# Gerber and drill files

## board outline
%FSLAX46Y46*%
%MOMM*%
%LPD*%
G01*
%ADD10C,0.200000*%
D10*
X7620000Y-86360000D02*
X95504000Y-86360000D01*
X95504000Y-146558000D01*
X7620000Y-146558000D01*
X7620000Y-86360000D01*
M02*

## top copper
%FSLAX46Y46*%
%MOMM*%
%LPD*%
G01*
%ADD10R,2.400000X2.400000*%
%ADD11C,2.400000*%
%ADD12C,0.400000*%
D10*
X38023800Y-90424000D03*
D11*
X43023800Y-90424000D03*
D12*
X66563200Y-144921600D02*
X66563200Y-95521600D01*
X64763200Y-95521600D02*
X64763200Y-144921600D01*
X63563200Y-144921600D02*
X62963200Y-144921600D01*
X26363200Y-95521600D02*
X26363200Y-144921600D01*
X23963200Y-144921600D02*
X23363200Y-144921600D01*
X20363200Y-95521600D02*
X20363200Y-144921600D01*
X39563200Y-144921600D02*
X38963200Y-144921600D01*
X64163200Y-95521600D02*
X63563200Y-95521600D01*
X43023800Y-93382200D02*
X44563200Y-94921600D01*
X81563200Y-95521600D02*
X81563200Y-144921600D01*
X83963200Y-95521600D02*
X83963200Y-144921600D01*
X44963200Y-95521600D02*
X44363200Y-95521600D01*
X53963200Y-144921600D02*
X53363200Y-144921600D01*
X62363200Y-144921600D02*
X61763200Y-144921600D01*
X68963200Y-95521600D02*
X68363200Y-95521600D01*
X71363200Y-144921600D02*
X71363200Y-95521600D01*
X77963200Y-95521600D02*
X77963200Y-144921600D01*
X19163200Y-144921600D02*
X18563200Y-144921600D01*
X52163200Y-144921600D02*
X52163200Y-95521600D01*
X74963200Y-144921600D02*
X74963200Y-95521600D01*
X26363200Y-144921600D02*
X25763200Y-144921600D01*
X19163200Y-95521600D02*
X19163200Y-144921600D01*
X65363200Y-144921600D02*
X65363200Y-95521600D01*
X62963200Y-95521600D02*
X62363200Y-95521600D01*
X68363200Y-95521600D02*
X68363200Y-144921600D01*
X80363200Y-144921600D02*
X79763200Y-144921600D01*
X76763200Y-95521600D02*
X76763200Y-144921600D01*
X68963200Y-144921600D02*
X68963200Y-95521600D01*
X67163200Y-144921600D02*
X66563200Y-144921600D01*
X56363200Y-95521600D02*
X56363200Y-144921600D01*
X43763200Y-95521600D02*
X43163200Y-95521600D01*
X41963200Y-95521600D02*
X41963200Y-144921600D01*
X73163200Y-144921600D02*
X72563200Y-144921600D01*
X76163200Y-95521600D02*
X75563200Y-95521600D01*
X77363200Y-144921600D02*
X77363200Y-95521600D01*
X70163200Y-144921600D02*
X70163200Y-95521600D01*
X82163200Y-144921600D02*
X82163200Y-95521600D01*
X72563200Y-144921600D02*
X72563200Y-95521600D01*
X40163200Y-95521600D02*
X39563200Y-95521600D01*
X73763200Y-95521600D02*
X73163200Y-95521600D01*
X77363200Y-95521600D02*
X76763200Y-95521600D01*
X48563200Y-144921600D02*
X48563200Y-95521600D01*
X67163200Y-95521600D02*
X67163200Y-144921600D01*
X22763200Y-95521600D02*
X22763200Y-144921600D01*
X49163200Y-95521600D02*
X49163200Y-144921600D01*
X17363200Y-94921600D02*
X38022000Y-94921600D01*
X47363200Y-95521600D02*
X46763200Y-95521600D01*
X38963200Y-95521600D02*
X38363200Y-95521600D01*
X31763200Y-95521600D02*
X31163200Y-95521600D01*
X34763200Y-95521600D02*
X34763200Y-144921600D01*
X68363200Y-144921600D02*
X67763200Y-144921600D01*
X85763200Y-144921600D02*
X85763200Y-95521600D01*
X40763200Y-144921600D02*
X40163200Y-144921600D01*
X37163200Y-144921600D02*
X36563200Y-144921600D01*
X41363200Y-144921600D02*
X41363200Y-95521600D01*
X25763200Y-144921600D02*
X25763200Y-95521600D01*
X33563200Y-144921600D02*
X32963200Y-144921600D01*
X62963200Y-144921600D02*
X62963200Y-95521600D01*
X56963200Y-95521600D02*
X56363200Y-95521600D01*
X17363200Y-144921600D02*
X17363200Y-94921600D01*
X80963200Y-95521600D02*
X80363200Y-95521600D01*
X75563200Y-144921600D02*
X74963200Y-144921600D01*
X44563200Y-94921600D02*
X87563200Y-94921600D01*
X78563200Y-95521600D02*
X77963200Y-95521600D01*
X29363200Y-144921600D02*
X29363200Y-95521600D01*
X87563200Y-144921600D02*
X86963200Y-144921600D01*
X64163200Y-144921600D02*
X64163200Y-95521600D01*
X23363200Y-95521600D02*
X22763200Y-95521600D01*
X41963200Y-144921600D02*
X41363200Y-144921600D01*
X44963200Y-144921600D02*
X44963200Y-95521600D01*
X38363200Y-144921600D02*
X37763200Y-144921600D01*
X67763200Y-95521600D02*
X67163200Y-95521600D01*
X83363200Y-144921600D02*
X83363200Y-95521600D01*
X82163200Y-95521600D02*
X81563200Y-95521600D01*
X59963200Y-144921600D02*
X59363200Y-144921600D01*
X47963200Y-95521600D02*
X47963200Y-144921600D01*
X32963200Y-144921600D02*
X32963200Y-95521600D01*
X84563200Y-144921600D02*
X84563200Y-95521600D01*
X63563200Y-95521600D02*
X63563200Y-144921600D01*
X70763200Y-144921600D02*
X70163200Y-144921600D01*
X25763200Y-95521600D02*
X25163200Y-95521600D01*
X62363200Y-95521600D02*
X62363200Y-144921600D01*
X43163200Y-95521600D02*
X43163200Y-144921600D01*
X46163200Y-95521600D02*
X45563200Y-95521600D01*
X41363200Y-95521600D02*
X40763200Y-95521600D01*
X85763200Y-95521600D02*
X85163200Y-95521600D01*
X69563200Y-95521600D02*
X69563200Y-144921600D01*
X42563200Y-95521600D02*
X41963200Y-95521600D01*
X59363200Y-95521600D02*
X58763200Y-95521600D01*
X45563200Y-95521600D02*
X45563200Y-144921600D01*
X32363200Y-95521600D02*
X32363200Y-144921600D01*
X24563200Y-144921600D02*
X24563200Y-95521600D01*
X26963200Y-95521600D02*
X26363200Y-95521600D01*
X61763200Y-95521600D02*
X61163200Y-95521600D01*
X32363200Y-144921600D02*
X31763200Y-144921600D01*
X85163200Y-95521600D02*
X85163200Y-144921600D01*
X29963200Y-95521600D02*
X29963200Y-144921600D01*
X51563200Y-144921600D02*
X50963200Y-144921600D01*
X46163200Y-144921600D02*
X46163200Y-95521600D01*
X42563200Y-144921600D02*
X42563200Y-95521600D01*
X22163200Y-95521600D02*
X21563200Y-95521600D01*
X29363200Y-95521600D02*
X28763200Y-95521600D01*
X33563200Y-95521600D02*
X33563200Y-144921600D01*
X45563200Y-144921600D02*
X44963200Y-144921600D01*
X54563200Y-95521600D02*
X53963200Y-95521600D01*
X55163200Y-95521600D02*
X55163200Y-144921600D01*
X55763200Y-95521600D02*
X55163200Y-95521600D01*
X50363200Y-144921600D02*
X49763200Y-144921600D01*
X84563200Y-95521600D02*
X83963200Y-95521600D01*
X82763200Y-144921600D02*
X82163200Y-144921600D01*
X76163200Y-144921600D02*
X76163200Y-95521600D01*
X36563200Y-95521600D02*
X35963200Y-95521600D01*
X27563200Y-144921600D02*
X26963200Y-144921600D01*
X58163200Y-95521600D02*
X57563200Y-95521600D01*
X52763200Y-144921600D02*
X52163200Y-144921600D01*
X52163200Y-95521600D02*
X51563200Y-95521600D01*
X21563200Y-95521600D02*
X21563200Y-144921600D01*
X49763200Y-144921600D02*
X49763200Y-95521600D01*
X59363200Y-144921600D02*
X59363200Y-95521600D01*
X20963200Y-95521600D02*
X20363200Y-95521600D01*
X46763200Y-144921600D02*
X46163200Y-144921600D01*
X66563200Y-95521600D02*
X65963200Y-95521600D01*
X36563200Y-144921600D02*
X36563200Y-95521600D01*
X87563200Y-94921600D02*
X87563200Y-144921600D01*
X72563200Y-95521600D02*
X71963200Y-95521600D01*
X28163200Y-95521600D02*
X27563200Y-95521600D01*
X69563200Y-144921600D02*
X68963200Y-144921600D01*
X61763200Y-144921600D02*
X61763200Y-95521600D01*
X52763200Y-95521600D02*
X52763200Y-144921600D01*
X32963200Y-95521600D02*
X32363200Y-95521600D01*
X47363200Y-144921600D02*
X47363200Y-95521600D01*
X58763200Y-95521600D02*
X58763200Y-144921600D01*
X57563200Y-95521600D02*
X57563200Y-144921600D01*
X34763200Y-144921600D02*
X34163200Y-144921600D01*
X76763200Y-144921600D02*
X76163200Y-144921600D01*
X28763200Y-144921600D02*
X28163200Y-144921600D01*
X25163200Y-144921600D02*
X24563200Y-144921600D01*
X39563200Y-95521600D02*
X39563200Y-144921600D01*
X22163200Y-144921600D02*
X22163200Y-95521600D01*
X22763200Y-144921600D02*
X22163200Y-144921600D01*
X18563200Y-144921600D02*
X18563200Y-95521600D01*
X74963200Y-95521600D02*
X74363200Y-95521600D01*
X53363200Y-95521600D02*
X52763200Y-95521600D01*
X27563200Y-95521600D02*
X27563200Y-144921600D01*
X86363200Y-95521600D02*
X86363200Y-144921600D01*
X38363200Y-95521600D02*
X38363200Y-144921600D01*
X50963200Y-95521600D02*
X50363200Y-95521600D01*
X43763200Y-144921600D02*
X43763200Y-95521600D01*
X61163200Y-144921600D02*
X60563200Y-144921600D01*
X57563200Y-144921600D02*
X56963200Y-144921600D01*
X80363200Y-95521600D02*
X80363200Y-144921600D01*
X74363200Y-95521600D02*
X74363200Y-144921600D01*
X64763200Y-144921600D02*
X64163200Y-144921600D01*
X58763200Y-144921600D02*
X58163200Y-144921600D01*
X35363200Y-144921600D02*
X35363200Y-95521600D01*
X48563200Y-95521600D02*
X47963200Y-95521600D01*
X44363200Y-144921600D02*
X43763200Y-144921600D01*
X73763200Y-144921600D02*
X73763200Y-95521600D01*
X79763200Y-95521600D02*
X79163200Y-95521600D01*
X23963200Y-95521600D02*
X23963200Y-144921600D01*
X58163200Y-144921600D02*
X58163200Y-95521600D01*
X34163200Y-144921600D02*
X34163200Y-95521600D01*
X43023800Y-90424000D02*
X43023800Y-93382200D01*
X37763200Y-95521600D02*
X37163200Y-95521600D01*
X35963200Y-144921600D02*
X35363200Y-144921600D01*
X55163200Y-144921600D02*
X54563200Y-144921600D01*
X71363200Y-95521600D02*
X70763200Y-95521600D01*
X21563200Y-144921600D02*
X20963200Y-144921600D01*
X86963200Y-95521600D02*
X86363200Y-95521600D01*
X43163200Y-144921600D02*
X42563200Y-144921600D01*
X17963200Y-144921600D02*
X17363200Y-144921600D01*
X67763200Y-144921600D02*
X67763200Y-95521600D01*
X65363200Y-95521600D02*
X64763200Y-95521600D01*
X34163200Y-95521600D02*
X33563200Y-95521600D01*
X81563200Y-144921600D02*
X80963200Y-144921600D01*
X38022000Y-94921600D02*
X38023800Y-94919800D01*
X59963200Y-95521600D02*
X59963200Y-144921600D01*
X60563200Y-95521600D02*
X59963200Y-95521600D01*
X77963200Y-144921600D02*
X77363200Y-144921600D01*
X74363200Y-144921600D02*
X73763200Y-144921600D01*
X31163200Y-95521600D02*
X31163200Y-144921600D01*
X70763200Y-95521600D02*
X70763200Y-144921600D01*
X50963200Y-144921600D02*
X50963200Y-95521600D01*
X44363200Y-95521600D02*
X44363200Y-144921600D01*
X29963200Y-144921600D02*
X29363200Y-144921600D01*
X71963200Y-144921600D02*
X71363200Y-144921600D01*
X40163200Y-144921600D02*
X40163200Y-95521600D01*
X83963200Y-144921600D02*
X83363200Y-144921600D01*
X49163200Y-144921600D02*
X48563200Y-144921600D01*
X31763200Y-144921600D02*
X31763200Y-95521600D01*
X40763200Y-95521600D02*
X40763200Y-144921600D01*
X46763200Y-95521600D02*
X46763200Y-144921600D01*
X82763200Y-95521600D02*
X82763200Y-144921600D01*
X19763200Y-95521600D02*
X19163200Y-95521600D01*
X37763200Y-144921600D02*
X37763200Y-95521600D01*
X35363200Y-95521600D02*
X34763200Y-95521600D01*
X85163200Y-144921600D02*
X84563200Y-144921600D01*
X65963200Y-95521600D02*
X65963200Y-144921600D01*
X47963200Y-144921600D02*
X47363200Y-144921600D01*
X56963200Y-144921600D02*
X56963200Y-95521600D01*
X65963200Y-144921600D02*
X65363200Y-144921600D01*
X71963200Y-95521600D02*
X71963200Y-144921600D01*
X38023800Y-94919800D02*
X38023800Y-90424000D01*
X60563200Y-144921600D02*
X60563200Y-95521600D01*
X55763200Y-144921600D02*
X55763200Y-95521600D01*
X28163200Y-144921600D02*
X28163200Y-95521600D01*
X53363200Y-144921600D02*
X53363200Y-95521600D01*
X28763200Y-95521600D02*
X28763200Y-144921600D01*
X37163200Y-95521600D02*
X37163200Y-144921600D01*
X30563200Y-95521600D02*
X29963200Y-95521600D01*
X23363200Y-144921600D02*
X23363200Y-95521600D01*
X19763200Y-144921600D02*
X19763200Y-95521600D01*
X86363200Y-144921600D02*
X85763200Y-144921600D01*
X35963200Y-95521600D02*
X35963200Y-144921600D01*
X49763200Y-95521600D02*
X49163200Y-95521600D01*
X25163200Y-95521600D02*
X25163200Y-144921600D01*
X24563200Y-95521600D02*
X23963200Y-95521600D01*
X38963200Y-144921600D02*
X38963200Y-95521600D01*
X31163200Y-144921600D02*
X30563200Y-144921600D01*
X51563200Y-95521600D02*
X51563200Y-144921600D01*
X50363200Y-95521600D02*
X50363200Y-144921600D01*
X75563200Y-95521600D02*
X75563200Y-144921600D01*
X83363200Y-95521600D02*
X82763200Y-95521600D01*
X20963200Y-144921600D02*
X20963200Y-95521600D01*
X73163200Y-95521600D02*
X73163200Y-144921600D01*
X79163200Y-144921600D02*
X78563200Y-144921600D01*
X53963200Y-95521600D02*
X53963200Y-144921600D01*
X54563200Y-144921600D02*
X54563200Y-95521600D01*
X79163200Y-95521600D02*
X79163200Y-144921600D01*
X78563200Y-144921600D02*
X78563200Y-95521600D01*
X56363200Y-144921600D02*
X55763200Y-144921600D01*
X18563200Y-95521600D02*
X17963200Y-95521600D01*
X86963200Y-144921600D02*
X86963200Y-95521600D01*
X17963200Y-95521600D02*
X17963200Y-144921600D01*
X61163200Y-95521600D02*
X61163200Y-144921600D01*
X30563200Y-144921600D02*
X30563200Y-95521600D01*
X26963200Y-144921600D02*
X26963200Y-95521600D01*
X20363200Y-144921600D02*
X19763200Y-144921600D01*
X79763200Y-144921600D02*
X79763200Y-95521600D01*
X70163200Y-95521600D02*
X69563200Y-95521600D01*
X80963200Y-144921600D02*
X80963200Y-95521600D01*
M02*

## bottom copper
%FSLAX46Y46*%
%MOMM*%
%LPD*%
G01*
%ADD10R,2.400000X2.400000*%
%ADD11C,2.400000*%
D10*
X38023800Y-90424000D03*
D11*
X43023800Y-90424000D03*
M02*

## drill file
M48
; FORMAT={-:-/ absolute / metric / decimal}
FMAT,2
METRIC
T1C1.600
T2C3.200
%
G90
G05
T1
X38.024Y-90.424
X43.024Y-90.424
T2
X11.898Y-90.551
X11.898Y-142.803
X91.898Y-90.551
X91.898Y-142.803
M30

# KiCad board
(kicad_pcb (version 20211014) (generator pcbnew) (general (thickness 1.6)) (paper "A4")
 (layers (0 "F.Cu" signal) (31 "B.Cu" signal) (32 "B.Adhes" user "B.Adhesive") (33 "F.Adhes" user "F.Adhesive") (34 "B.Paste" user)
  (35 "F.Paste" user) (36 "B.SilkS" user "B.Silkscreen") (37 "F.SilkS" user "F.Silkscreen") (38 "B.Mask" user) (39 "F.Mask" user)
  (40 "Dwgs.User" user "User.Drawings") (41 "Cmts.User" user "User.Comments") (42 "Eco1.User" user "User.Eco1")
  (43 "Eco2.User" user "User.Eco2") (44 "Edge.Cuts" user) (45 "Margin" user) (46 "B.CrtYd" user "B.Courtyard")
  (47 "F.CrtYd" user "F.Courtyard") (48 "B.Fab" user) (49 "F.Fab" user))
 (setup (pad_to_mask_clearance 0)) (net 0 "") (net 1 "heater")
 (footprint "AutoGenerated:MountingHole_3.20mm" (layer "F.Cu") (at 91.898 142.803)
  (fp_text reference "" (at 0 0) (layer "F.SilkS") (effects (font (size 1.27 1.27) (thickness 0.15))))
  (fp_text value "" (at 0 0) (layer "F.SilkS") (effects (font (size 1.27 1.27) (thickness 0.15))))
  (pad "" np_thru_hole circle locked (at 0 0) (size 3.2 3.2) (drill 3.2) (layers *.Cu *.Mask)))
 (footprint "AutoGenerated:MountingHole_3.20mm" (layer "F.Cu") (at 11.898 90.551)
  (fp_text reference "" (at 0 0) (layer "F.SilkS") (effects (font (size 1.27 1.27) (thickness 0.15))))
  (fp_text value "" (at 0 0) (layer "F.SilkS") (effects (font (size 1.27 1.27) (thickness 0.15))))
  (pad "" np_thru_hole circle locked (at 0 0) (size 3.2 3.2) (drill 3.2) (layers *.Cu *.Mask)))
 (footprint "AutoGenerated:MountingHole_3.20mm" (layer "F.Cu") (at 91.898 90.551)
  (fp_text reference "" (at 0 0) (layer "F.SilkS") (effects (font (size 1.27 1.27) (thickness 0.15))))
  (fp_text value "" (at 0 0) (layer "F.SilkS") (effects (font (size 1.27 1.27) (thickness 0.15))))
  (pad "" np_thru_hole circle locked (at 0 0) (size 3.2 3.2) (drill 3.2) (layers *.Cu *.Mask)))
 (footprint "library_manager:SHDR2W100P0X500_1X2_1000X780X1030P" (layer "F.Cu") (at 38.0238 90.424)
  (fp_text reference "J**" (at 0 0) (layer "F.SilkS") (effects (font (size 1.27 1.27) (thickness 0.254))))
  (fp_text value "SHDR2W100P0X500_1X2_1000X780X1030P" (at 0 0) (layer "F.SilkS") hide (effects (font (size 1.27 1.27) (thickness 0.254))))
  (pad "1" thru_hole rect locked (at 0 0) (size 2.4 2.4) (drill 1.6) (layers *.Cu *.Mask) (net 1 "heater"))
  (pad "2" thru_hole circle locked (at 5 0) (size 2.4 2.4) (drill 1.6) (layers *.Cu *.Mask) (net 1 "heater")))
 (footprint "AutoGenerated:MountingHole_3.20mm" (layer "F.Cu") (at 11.898 142.803)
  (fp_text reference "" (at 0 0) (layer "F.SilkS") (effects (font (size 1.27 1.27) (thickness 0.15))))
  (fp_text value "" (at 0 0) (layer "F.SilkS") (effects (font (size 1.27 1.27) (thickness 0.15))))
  (pad "" np_thru_hole circle locked (at 0 0) (size 3.2 3.2) (drill 3.2) (layers *.Cu *.Mask)))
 (gr_rect (start 7.62 86.36) (end 95.504 146.558) (layer "Edge.Cuts") (width 0.2) (fill none))
 (segment (start 66.5632 144.9216) (end 66.5632 95.5216) (width 0.4) (layer "F.Cu") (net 1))
 (segment (start 64.7632 95.5216) (end 64.7632 144.9216) (width 0.4) (layer "F.Cu") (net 1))
 (segment (start 63.5632 144.9216) (end 62.9632 144.9216) (width 0.4) (layer "F.Cu") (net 1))
 (segment (start 26.3632 95.5216) (end 26.3632 144.9216) (width 0.4) (layer "F.Cu") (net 1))
 (segment (start 23.9632 144.9216) (end 23.3632 144.9216) (width 0.4) (layer "F.Cu") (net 1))
 (segment (start 20.3632 95.5216) (end 20.3632 144.9216) (width 0.4) (layer "F.Cu") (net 1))
 (segment (start 39.5632 144.9216) (end 38.9632 144.9216) (width 0.4) (layer "F.Cu") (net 1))
 (segment (start 64.1632 95.5216) (end 63.5632 95.5216) (width 0.4) (layer "F.Cu") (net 1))
 (segment (start 43.0238 93.3822) (end 44.5632 94.9216) (width 0.4) (layer "F.Cu") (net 1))
 (segment (start 81.5632 95.5216) (end 81.5632 144.9216) (width 0.4) (layer "F.Cu") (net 1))
 (segment (start 83.9632 95.5216) (end 83.9632 144.9216) (width 0.4) (layer "F.Cu") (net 1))
 (segment (start 44.9632 95.5216) (end 44.3632 95.5216) (width 0.4) (layer "F.Cu") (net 1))
 (segment (start 53.9632 144.9216) (end 53.3632 144.9216) (width 0.4) (layer "F.Cu") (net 1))
 (segment (start 62.3632 144.9216) (end 61.7632 144.9216) (width 0.4) (layer "F.Cu") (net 1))
 (segment (start 68.9632 95.5216) (end 68.3632 95.5216) (width 0.4) (layer "F.Cu") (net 1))
 (segment (start 71.3632 144.9216) (end 71.3632 95.5216) (width 0.4) (layer "F.Cu") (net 1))
 (segment (start 77.9632 95.5216) (end 77.9632 144.9216) (width 0.4) (layer "F.Cu") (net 1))
 (segment (start 19.1632 144.9216) (end 18.5632 144.9216) (width 0.4) (layer "F.Cu") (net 1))
 (segment (start 52.1632 144.9216) (end 52.1632 95.5216) (width 0.4) (layer "F.Cu") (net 1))
 (segment (start 74.9632 144.9216) (end 74.9632 95.5216) (width 0.4) (layer "F.Cu") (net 1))
 (segment (start 26.3632 144.9216) (end 25.7632 144.9216) (width 0.4) (layer "F.Cu") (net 1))
 (segment (start 19.1632 95.5216) (end 19.1632 144.9216) (width 0.4) (layer "F.Cu") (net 1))
 (segment (start 65.3632 144.9216) (end 65.3632 95.5216) (width 0.4) (layer "F.Cu") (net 1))
 (segment (start 62.9632 95.5216) (end 62.3632 95.5216) (width 0.4) (layer "F.Cu") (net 1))
 (segment (start 68.3632 95.5216) (end 68.3632 144.9216) (width 0.4) (layer "F.Cu") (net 1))
 (segment (start 80.3632 144.9216) (end 79.7632 144.9216) (width 0.4) (layer "F.Cu") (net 1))
 (segment (start 76.7632 95.5216) (end 76.7632 144.9216) (width 0.4) (layer "F.Cu") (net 1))
 (segment (start 68.9632 144.9216) (end 68.9632 95.5216) (width 0.4) (layer "F.Cu") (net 1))
 (segment (start 67.1632 144.9216) (end 66.5632 144.9216) (width 0.4) (layer "F.Cu") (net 1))
 (segment (start 56.3632 95.5216) (end 56.3632 144.9216) (width 0.4) (layer "F.Cu") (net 1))
 (segment (start 43.7632 95.5216) (end 43.1632 95.5216) (width 0.4) (layer "F.Cu") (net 1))
 (segment (start 41.9632 95.5216) (end 41.9632 144.9216) (width 0.4) (layer "F.Cu") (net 1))
 (segment (start 73.1632 144.9216) (end 72.5632 144.9216) (width 0.4) (layer "F.Cu") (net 1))
 (segment (start 76.1632 95.5216) (end 75.5632 95.5216) (width 0.4) (layer "F.Cu") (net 1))
 (segment (start 77.3632 144.9216) (end 77.3632 95.5216) (width 0.4) (layer "F.Cu") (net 1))
 (segment (start 70.1632 144.9216) (end 70.1632 95.5216) (width 0.4) (layer "F.Cu") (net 1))
 (segment (start 82.1632 144.9216) (end 82.1632 95.5216) (width 0.4) (layer "F.Cu") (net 1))
 (segment (start 72.5632 144.9216) (end 72.5632 95.5216) (width 0.4) (layer "F.Cu") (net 1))
 (segment (start 40.1632 95.5216) (end 39.5632 95.5216) (width 0.4) (layer "F.Cu") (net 1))
 (segment (start 73.7632 95.5216) (end 73.1632 95.5216) (width 0.4) (layer "F.Cu") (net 1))
 (segment (start 77.3632 95.5216) (end 76.7632 95.5216) (width 0.4) (layer "F.Cu") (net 1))
 (segment (start 48.5632 144.9216) (end 48.5632 95.5216) (width 0.4) (layer "F.Cu") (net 1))
 (segment (start 67.1632 95.5216) (end 67.1632 144.9216) (width 0.4) (layer "F.Cu") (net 1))
 (segment (start 22.7632 95.5216) (end 22.7632 144.9216) (width 0.4) (layer "F.Cu") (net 1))
 (segment (start 49.1632 95.5216) (end 49.1632 144.9216) (width 0.4) (layer "F.Cu") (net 1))
 (segment (start 17.3632 94.9216) (end 38.022 94.9216) (width 0.4) (layer "F.Cu") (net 1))
 (segment (start 47.3632 95.5216) (end 46.7632 95.5216) (width 0.4) (layer "F.Cu") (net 1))
 (segment (start 38.9632 95.5216) (end 38.3632 95.5216) (width 0.4) (layer "F.Cu") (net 1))
 (segment (start 31.7632 95.5216) (end 31.1632 95.5216) (width 0.4) (layer "F.Cu") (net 1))
 (segment (start 34.7632 95.5216) (end 34.7632 144.9216) (width 0.4) (layer "F.Cu") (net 1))
 (segment (start 68.3632 144.9216) (end 67.7632 144.9216) (width 0.4) (layer "F.Cu") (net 1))
 (segment (start 85.7632 144.9216) (end 85.7632 95.5216) (width 0.4) (layer "F.Cu") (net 1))
 (segment (start 40.7632 144.9216) (end 40.1632 144.9216) (width 0.4) (layer "F.Cu") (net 1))
 (segment (start 37.1632 144.9216) (end 36.5632 144.9216) (width 0.4) (layer "F.Cu") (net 1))
 (segment (start 41.3632 144.9216) (end 41.3632 95.5216) (width 0.4) (layer "F.Cu") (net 1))
 (segment (start 25.7632 144.9216) (end 25.7632 95.5216) (width 0.4) (layer "F.Cu") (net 1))
 (segment (start 33.5632 144.9216) (end 32.9632 144.9216) (width 0.4) (layer "F.Cu") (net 1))
 (segment (start 62.9632 144.9216) (end 62.9632 95.5216) (width 0.4) (layer "F.Cu") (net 1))
 (segment (start 56.9632 95.5216) (end 56.3632 95.5216) (width 0.4) (layer "F.Cu") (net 1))
 (segment (start 17.3632 144.9216) (end 17.3632 94.9216) (width 0.4) (layer "F.Cu") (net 1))
 (segment (start 80.9632 95.5216) (end 80.3632 95.5216) (width 0.4) (layer "F.Cu") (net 1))
 (segment (start 75.5632 144.9216) (end 74.9632 144.9216) (width 0.4) (layer "F.Cu") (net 1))
 (segment (start 44.5632 94.9216) (end 87.5632 94.9216) (width 0.4) (layer "F.Cu") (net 1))
 (segment (start 78.5632 95.5216) (end 77.9632 95.5216) (width 0.4) (layer "F.Cu") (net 1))
 (segment (start 29.3632 144.9216) (end 29.3632 95.5216) (width 0.4) (layer "F.Cu") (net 1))
 (segment (start 87.5632 144.9216) (end 86.9632 144.9216) (width 0.4) (layer "F.Cu") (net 1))
 (segment (start 64.1632 144.9216) (end 64.1632 95.5216) (width 0.4) (layer "F.Cu") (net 1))
 (segment (start 23.3632 95.5216) (end 22.7632 95.5216) (width 0.4) (layer "F.Cu") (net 1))
 (segment (start 41.9632 144.9216) (end 41.3632 144.9216) (width 0.4) (layer "F.Cu") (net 1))
 (segment (start 44.9632 144.9216) (end 44.9632 95.5216) (width 0.4) (layer "F.Cu") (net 1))
 (segment (start 38.3632 144.9216) (end 37.7632 144.9216) (width 0.4) (layer "F.Cu") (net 1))
 (segment (start 67.7632 95.5216) (end 67.1632 95.5216) (width 0.4) (layer "F.Cu") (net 1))
 (segment (start 83.3632 144.9216) (end 83.3632 95.5216) (width 0.4) (layer "F.Cu") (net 1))
 (segment (start 82.1632 95.5216) (end 81.5632 95.5216) (width 0.4) (layer "F.Cu") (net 1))
 (segment (start 59.9632 144.9216) (end 59.3632 144.9216) (width 0.4) (layer "F.Cu") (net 1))
 (segment (start 47.9632 95.5216) (end 47.9632 144.9216) (width 0.4) (layer "F.Cu") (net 1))
 (segment (start 32.9632 144.9216) (end 32.9632 95.5216) (width 0.4) (layer "F.Cu") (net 1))
 (segment (start 84.5632 144.9216) (end 84.5632 95.5216) (width 0.4) (layer "F.Cu") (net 1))
 (segment (start 63.5632 95.5216) (end 63.5632 144.9216) (width 0.4) (layer "F.Cu") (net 1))
 (segment (start 70.7632 144.9216) (end 70.1632 144.9216) (width 0.4) (layer "F.Cu") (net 1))
 (segment (start 25.7632 95.5216) (end 25.1632 95.5216) (width 0.4) (layer "F.Cu") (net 1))
 (segment (start 62.3632 95.5216) (end 62.3632 144.9216) (width 0.4) (layer "F.Cu") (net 1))
 (segment (start 43.1632 95.5216) (end 43.1632 144.9216) (width 0.4) (layer "F.Cu") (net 1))
 (segment (start 46.1632 95.5216) (end 45.5632 95.5216) (width 0.4) (layer "F.Cu") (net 1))
 (segment (start 41.3632 95.5216) (end 40.7632 95.5216) (width 0.4) (layer "F.Cu") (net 1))
 (segment (start 85.7632 95.5216) (end 85.1632 95.5216) (width 0.4) (layer "F.Cu") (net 1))
 (segment (start 69.5632 95.5216) (end 69.5632 144.9216) (width 0.4) (layer "F.Cu") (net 1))
 (segment (start 42.5632 95.5216) (end 41.9632 95.5216) (width 0.4) (layer "F.Cu") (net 1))
 (segment (start 59.3632 95.5216) (end 58.7632 95.5216) (width 0.4) (layer "F.Cu") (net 1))
 (segment (start 45.5632 95.5216) (end 45.5632 144.9216) (width 0.4) (layer "F.Cu") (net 1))
 (segment (start 32.3632 95.5216) (end 32.3632 144.9216) (width 0.4) (layer "F.Cu") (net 1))
 (segment (start 24.5632 144.9216) (end 24.5632 95.5216) (width 0.4) (layer "F.Cu") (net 1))
 (segment (start 26.9632 95.5216) (end 26.3632 95.5216) (width 0.4) (layer "F.Cu") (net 1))
 (segment (start 61.7632 95.5216) (end 61.1632 95.5216) (width 0.4) (layer "F.Cu") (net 1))
 (segment (start 32.3632 144.9216) (end 31.7632 144.9216) (width 0.4) (layer "F.Cu") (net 1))
 (segment (start 85.1632 95.5216) (end 85.1632 144.9216) (width 0.4) (layer "F.Cu") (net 1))
 (segment (start 29.9632 95.5216) (end 29.9632 144.9216) (width 0.4) (layer "F.Cu") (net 1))
 (segment (start 51.5632 144.9216) (end 50.9632 144.9216) (width 0.4) (layer "F.Cu") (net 1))
 (segment (start 46.1632 144.9216) (end 46.1632 95.5216) (width 0.4) (layer "F.Cu") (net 1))
 (segment (start 42.5632 144.9216) (end 42.5632 95.5216) (width 0.4) (layer "F.Cu") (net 1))
 (segment (start 22.1632 95.5216) (end 21.5632 95.5216) (width 0.4) (layer "F.Cu") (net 1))
 (segment (start 29.3632 95.5216) (end 28.7632 95.5216) (width 0.4) (layer "F.Cu") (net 1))
 (segment (start 33.5632 95.5216) (end 33.5632 144.9216) (width 0.4) (layer "F.Cu") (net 1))
 (segment (start 45.5632 144.9216) (end 44.9632 144.9216) (width 0.4) (layer "F.Cu") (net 1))
 (segment (start 54.5632 95.5216) (end 53.9632 95.5216) (width 0.4) (layer "F.Cu") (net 1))
 (segment (start 55.1632 95.5216) (end 55.1632 144.9216) (width 0.4) (layer "F.Cu") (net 1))
 (segment (start 55.7632 95.5216) (end 55.1632 95.5216) (width 0.4) (layer "F.Cu") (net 1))
 (segment (start 50.3632 144.9216) (end 49.7632 144.9216) (width 0.4) (layer "F.Cu") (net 1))
 (segment (start 84.5632 95.5216) (end 83.9632 95.5216) (width 0.4) (layer "F.Cu") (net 1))
 (segment (start 82.7632 144.9216) (end 82.1632 144.9216) (width 0.4) (layer "F.Cu") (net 1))
 (segment (start 76.1632 144.9216) (end 76.1632 95.5216) (width 0.4) (layer "F.Cu") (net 1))
 (segment (start 36.5632 95.5216) (end 35.9632 95.5216) (width 0.4) (layer "F.Cu") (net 1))
 (segment (start 27.5632 144.9216) (end 26.9632 144.9216) (width 0.4) (layer "F.Cu") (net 1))
 (segment (start 58.1632 95.5216) (end 57.5632 95.5216) (width 0.4) (layer "F.Cu") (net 1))
 (segment (start 52.7632 144.9216) (end 52.1632 144.9216) (width 0.4) (layer "F.Cu") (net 1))
 (segment (start 52.1632 95.5216) (end 51.5632 95.5216) (width 0.4) (layer "F.Cu") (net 1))
 (segment (start 21.5632 95.5216) (end 21.5632 144.9216) (width 0.4) (layer "F.Cu") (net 1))
 (segment (start 49.7632 144.9216) (end 49.7632 95.5216) (width 0.4) (layer "F.Cu") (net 1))
 (segment (start 59.3632 144.9216) (end 59.3632 95.5216) (width 0.4) (layer "F.Cu") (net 1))
 (segment (start 20.9632 95.5216) (end 20.3632 95.5216) (width 0.4) (layer "F.Cu") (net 1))
 (segment (start 46.7632 144.9216) (end 46.1632 144.9216) (width 0.4) (layer "F.Cu") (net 1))
 (segment (start 66.5632 95.5216) (end 65.9632 95.5216) (width 0.4) (layer "F.Cu") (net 1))
 (segment (start 36.5632 144.9216) (end 36.5632 95.5216) (width 0.4) (layer "F.Cu") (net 1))
 (segment (start 87.5632 94.9216) (end 87.5632 144.9216) (width 0.4) (layer "F.Cu") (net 1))
 (segment (start 72.5632 95.5216) (end 71.9632 95.5216) (width 0.4) (layer "F.Cu") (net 1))
 (segment (start 28.1632 95.5216) (end 27.5632 95.5216) (width 0.4) (layer "F.Cu") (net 1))
 (segment (start 69.5632 144.9216) (end 68.9632 144.9216) (width 0.4) (layer "F.Cu") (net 1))
 (segment (start 61.7632 144.9216) (end 61.7632 95.5216) (width 0.4) (layer "F.Cu") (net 1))
 (segment (start 52.7632 95.5216) (end 52.7632 144.9216) (width 0.4) (layer "F.Cu") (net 1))
 (segment (start 32.9632 95.5216) (end 32.3632 95.5216) (width 0.4) (layer "F.Cu") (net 1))
 (segment (start 47.3632 144.9216) (end 47.3632 95.5216) (width 0.4) (layer "F.Cu") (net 1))
 (segment (start 58.7632 95.5216) (end 58.7632 144.9216) (width 0.4) (layer "F.Cu") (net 1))
 (segment (start 57.5632 95.5216) (end 57.5632 144.9216) (width 0.4) (layer "F.Cu") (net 1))
 (segment (start 34.7632 144.9216) (end 34.1632 144.9216) (width 0.4) (layer "F.Cu") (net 1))
 (segment (start 76.7632 144.9216) (end 76.1632 144.9216) (width 0.4) (layer "F.Cu") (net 1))
 (segment (start 28.7632 144.9216) (end 28.1632 144.9216) (width 0.4) (layer "F.Cu") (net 1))
 (segment (start 25.1632 144.9216) (end 24.5632 144.9216) (width 0.4) (layer "F.Cu") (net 1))
 (segment (start 39.5632 95.5216) (end 39.5632 144.9216) (width 0.4) (layer "F.Cu") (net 1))
 (segment (start 22.1632 144.9216) (end 22.1632 95.5216) (width 0.4) (layer "F.Cu") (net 1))
 (segment (start 22.7632 144.9216) (end 22.1632 144.9216) (width 0.4) (layer "F.Cu") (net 1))
 (segment (start 18.5632 144.9216) (end 18.5632 95.5216) (width 0.4) (layer "F.Cu") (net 1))
 (segment (start 74.9632 95.5216) (end 74.3632 95.5216) (width 0.4) (layer "F.Cu") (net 1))
 (segment (start 53.3632 95.5216) (end 52.7632 95.5216) (width 0.4) (layer "F.Cu") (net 1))
 (segment (start 27.5632 95.5216) (end 27.5632 144.9216) (width 0.4) (layer "F.Cu") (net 1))
 (segment (start 86.3632 95.5216) (end 86.3632 144.9216) (width 0.4) (layer "F.Cu") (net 1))
 (segment (start 38.3632 95.5216) (end 38.3632 144.9216) (width 0.4) (layer "F.Cu") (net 1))
 (segment (start 50.9632 95.5216) (end 50.3632 95.5216) (width 0.4) (layer "F.Cu") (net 1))
 (segment (start 43.7632 144.9216) (end 43.7632 95.5216) (width 0.4) (layer "F.Cu") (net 1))
 (segment (start 61.1632 144.9216) (end 60.5632 144.9216) (width 0.4) (layer "F.Cu") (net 1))
 (segment (start 57.5632 144.9216) (end 56.9632 144.9216) (width 0.4) (layer "F.Cu") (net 1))
 (segment (start 80.3632 95.5216) (end 80.3632 144.9216) (width 0.4) (layer "F.Cu") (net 1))
 (segment (start 74.3632 95.5216) (end 74.3632 144.9216) (width 0.4) (layer "F.Cu") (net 1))
 (segment (start 64.7632 144.9216) (end 64.1632 144.9216) (width 0.4) (layer "F.Cu") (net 1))
 (segment (start 58.7632 144.9216) (end 58.1632 144.9216) (width 0.4) (layer "F.Cu") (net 1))
 (segment (start 35.3632 144.9216) (end 35.3632 95.5216) (width 0.4) (layer "F.Cu") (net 1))
 (segment (start 48.5632 95.5216) (end 47.9632 95.5216) (width 0.4) (layer "F.Cu") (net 1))
 (segment (start 44.3632 144.9216) (end 43.7632 144.9216) (width 0.4) (layer "F.Cu") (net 1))
 (segment (start 73.7632 144.9216) (end 73.7632 95.5216) (width 0.4) (layer "F.Cu") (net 1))
 (segment (start 79.7632 95.5216) (end 79.1632 95.5216) (width 0.4) (layer "F.Cu") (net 1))
 (segment (start 23.9632 95.5216) (end 23.9632 144.9216) (width 0.4) (layer "F.Cu") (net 1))
 (segment (start 58.1632 144.9216) (end 58.1632 95.5216) (width 0.4) (layer "F.Cu") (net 1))
 (segment (start 34.1632 144.9216) (end 34.1632 95.5216) (width 0.4) (layer "F.Cu") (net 1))
 (segment (start 43.0238 90.424) (end 43.0238 93.3822) (width 0.4) (layer "F.Cu") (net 1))
 (segment (start 37.7632 95.5216) (end 37.1632 95.5216) (width 0.4) (layer "F.Cu") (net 1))
 (segment (start 35.9632 144.9216) (end 35.3632 144.9216) (width 0.4) (layer "F.Cu") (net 1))
 (segment (start 55.1632 144.9216) (end 54.5632 144.9216) (width 0.4) (layer "F.Cu") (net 1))
 (segment (start 71.3632 95.5216) (end 70.7632 95.5216) (width 0.4) (layer "F.Cu") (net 1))
 (segment (start 21.5632 144.9216) (end 20.9632 144.9216) (width 0.4) (layer "F.Cu") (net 1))
 (segment (start 86.9632 95.5216) (end 86.3632 95.5216) (width 0.4) (layer "F.Cu") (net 1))
 (segment (start 43.1632 144.9216) (end 42.5632 144.9216) (width 0.4) (layer "F.Cu") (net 1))
 (segment (start 17.9632 144.9216) (end 17.3632 144.9216) (width 0.4) (layer "F.Cu") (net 1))
 (segment (start 67.7632 144.9216) (end 67.7632 95.5216) (width 0.4) (layer "F.Cu") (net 1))
 (segment (start 65.3632 95.5216) (end 64.7632 95.5216) (width 0.4) (layer "F.Cu") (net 1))
 (segment (start 34.1632 95.5216) (end 33.5632 95.5216) (width 0.4) (layer "F.Cu") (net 1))
 (segment (start 81.5632 144.9216) (end 80.9632 144.9216) (width 0.4) (layer "F.Cu") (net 1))
 (segment (start 38.022 94.9216) (end 38.0238 94.9198) (width 0.4) (layer "F.Cu") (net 1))
 (segment (start 59.9632 95.5216) (end 59.9632 144.9216) (width 0.4) (layer "F.Cu") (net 1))
 (segment (start 60.5632 95.5216) (end 59.9632 95.5216) (width 0.4) (layer "F.Cu") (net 1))
 (segment (start 77.9632 144.9216) (end 77.3632 144.9216) (width 0.4) (layer "F.Cu") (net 1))
 (segment (start 74.3632 144.9216) (end 73.7632 144.9216) (width 0.4) (layer "F.Cu") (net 1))
 (segment (start 31.1632 95.5216) (end 31.1632 144.9216) (width 0.4) (layer "F.Cu") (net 1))
 (segment (start 70.7632 95.5216) (end 70.7632 144.9216) (width 0.4) (layer "F.Cu") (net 1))
 (segment (start 50.9632 144.9216) (end 50.9632 95.5216) (width 0.4) (layer "F.Cu") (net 1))
 (segment (start 44.3632 95.5216) (end 44.3632 144.9216) (width 0.4) (layer "F.Cu") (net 1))
 (segment (start 29.9632 144.9216) (end 29.3632 144.9216) (width 0.4) (layer "F.Cu") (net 1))
 (segment (start 71.9632 144.9216) (end 71.3632 144.9216) (width 0.4) (layer "F.Cu") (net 1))
 (segment (start 40.1632 144.9216) (end 40.1632 95.5216) (width 0.4) (layer "F.Cu") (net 1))
 (segment (start 83.9632 144.9216) (end 83.3632 144.9216) (width 0.4) (layer "F.Cu") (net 1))
 (segment (start 49.1632 144.9216) (end 48.5632 144.9216) (width 0.4) (layer "F.Cu") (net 1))
 (segment (start 31.7632 144.9216) (end 31.7632 95.5216) (width 0.4) (layer "F.Cu") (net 1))
 (segment (start 40.7632 95.5216) (end 40.7632 144.9216) (width 0.4) (layer "F.Cu") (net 1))
 (segment (start 46.7632 95.5216) (end 46.7632 144.9216) (width 0.4) (layer "F.Cu") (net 1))
 (segment (start 82.7632 95.5216) (end 82.7632 144.9216) (width 0.4) (layer "F.Cu") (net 1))
 (segment (start 19.7632 95.5216) (end 19.1632 95.5216) (width 0.4) (layer "F.Cu") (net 1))
 (segment (start 37.7632 144.9216) (end 37.7632 95.5216) (width 0.4) (layer "F.Cu") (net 1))
 (segment (start 35.3632 95.5216) (end 34.7632 95.5216) (width 0.4) (layer "F.Cu") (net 1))
 (segment (start 85.1632 144.9216) (end 84.5632 144.9216) (width 0.4) (layer "F.Cu") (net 1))
 (segment (start 65.9632 95.5216) (end 65.9632 144.9216) (width 0.4) (layer "F.Cu") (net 1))
 (segment (start 47.9632 144.9216) (end 47.3632 144.9216) (width 0.4) (layer "F.Cu") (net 1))
 (segment (start 56.9632 144.9216) (end 56.9632 95.5216) (width 0.4) (layer "F.Cu") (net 1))
 (segment (start 65.9632 144.9216) (end 65.3632 144.9216) (width 0.4) (layer "F.Cu") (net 1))
 (segment (start 71.9632 95.5216) (end 71.9632 144.9216) (width 0.4) (layer "F.Cu") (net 1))
 (segment (start 38.0238 94.9198) (end 38.0238 90.424) (width 0.4) (layer "F.Cu") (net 1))
 (segment (start 60.5632 144.9216) (end 60.5632 95.5216) (width 0.4) (layer "F.Cu") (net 1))
 (segment (start 55.7632 144.9216) (end 55.7632 95.5216) (width 0.4) (layer "F.Cu") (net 1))
 (segment (start 28.1632 144.9216) (end 28.1632 95.5216) (width 0.4) (layer "F.Cu") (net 1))
 (segment (start 53.3632 144.9216) (end 53.3632 95.5216) (width 0.4) (layer "F.Cu") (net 1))
 (segment (start 28.7632 95.5216) (end 28.7632 144.9216) (width 0.4) (layer "F.Cu") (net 1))
 (segment (start 37.1632 95.5216) (end 37.1632 144.9216) (width 0.4) (layer "F.Cu") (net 1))
 (segment (start 30.5632 95.5216) (end 29.9632 95.5216) (width 0.4) (layer "F.Cu") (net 1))
 (segment (start 23.3632 144.9216) (end 23.3632 95.5216) (width 0.4) (layer "F.Cu") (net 1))
 (segment (start 19.7632 144.9216) (end 19.7632 95.5216) (width 0.4) (layer "F.Cu") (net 1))
 (segment (start 86.3632 144.9216) (end 85.7632 144.9216) (width 0.4) (layer "F.Cu") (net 1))
 (segment (start 35.9632 95.5216) (end 35.9632 144.9216) (width 0.4) (layer "F.Cu") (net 1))
 (segment (start 49.7632 95.5216) (end 49.1632 95.5216) (width 0.4) (layer "F.Cu") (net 1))
 (segment (start 25.1632 95.5216) (end 25.1632 144.9216) (width 0.4) (layer "F.Cu") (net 1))
 (segment (start 24.5632 95.5216) (end 23.9632 95.5216) (width 0.4) (layer "F.Cu") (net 1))
 (segment (start 38.9632 144.9216) (end 38.9632 95.5216) (width 0.4) (layer "F.Cu") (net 1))
 (segment (start 31.1632 144.9216) (end 30.5632 144.9216) (width 0.4) (layer "F.Cu") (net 1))
 (segment (start 51.5632 95.5216) (end 51.5632 144.9216) (width 0.4) (layer "F.Cu") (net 1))
 (segment (start 50.3632 95.5216) (end 50.3632 144.9216) (width 0.4) (layer "F.Cu") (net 1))
 (segment (start 75.5632 95.5216) (end 75.5632 144.9216) (width 0.4) (layer "F.Cu") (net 1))
 (segment (start 83.3632 95.5216) (end 82.7632 95.5216) (width 0.4) (layer "F.Cu") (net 1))
 (segment (start 20.9632 144.9216) (end 20.9632 95.5216) (width 0.4) (layer "F.Cu") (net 1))
 (segment (start 73.1632 95.5216) (end 73.1632 144.9216) (width 0.4) (layer "F.Cu") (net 1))
 (segment (start 79.1632 144.9216) (end 78.5632 144.9216) (width 0.4) (layer "F.Cu") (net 1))
 (segment (start 53.9632 95.5216) (end 53.9632 144.9216) (width 0.4) (layer "F.Cu") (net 1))
 (segment (start 54.5632 144.9216) (end 54.5632 95.5216) (width 0.4) (layer "F.Cu") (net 1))
 (segment (start 79.1632 95.5216) (end 79.1632 144.9216) (width 0.4) (layer "F.Cu") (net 1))
 (segment (start 78.5632 144.9216) (end 78.5632 95.5216) (width 0.4) (layer "F.Cu") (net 1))
 (segment (start 56.3632 144.9216) (end 55.7632 144.9216) (width 0.4) (layer "F.Cu") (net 1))
 (segment (start 18.5632 95.5216) (end 17.9632 95.5216) (width 0.4) (layer "F.Cu") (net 1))
 (segment (start 86.9632 144.9216) (end 86.9632 95.5216) (width 0.4) (layer "F.Cu") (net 1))
 (segment (start 17.9632 95.5216) (end 17.9632 144.9216) (width 0.4) (layer "F.Cu") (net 1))
 (segment (start 61.1632 95.5216) (end 61.1632 144.9216) (width 0.4) (layer "F.Cu") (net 1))
 (segment (start 30.5632 144.9216) (end 30.5632 95.5216) (width 0.4) (layer "F.Cu") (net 1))
 (segment (start 26.9632 144.9216) (end 26.9632 95.5216) (width 0.4) (layer "F.Cu") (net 1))
 (segment (start 20.3632 144.9216) (end 19.7632 144.9216) (width 0.4) (layer "F.Cu") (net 1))
 (segment (start 79.7632 144.9216) (end 79.7632 95.5216) (width 0.4) (layer "F.Cu") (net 1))
 (segment (start 70.1632 95.5216) (end 69.5632 95.5216) (width 0.4) (layer "F.Cu") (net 1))
 (segment (start 80.9632 144.9216) (end 80.9632 95.5216) (width 0.4) (layer "F.Cu") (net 1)))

